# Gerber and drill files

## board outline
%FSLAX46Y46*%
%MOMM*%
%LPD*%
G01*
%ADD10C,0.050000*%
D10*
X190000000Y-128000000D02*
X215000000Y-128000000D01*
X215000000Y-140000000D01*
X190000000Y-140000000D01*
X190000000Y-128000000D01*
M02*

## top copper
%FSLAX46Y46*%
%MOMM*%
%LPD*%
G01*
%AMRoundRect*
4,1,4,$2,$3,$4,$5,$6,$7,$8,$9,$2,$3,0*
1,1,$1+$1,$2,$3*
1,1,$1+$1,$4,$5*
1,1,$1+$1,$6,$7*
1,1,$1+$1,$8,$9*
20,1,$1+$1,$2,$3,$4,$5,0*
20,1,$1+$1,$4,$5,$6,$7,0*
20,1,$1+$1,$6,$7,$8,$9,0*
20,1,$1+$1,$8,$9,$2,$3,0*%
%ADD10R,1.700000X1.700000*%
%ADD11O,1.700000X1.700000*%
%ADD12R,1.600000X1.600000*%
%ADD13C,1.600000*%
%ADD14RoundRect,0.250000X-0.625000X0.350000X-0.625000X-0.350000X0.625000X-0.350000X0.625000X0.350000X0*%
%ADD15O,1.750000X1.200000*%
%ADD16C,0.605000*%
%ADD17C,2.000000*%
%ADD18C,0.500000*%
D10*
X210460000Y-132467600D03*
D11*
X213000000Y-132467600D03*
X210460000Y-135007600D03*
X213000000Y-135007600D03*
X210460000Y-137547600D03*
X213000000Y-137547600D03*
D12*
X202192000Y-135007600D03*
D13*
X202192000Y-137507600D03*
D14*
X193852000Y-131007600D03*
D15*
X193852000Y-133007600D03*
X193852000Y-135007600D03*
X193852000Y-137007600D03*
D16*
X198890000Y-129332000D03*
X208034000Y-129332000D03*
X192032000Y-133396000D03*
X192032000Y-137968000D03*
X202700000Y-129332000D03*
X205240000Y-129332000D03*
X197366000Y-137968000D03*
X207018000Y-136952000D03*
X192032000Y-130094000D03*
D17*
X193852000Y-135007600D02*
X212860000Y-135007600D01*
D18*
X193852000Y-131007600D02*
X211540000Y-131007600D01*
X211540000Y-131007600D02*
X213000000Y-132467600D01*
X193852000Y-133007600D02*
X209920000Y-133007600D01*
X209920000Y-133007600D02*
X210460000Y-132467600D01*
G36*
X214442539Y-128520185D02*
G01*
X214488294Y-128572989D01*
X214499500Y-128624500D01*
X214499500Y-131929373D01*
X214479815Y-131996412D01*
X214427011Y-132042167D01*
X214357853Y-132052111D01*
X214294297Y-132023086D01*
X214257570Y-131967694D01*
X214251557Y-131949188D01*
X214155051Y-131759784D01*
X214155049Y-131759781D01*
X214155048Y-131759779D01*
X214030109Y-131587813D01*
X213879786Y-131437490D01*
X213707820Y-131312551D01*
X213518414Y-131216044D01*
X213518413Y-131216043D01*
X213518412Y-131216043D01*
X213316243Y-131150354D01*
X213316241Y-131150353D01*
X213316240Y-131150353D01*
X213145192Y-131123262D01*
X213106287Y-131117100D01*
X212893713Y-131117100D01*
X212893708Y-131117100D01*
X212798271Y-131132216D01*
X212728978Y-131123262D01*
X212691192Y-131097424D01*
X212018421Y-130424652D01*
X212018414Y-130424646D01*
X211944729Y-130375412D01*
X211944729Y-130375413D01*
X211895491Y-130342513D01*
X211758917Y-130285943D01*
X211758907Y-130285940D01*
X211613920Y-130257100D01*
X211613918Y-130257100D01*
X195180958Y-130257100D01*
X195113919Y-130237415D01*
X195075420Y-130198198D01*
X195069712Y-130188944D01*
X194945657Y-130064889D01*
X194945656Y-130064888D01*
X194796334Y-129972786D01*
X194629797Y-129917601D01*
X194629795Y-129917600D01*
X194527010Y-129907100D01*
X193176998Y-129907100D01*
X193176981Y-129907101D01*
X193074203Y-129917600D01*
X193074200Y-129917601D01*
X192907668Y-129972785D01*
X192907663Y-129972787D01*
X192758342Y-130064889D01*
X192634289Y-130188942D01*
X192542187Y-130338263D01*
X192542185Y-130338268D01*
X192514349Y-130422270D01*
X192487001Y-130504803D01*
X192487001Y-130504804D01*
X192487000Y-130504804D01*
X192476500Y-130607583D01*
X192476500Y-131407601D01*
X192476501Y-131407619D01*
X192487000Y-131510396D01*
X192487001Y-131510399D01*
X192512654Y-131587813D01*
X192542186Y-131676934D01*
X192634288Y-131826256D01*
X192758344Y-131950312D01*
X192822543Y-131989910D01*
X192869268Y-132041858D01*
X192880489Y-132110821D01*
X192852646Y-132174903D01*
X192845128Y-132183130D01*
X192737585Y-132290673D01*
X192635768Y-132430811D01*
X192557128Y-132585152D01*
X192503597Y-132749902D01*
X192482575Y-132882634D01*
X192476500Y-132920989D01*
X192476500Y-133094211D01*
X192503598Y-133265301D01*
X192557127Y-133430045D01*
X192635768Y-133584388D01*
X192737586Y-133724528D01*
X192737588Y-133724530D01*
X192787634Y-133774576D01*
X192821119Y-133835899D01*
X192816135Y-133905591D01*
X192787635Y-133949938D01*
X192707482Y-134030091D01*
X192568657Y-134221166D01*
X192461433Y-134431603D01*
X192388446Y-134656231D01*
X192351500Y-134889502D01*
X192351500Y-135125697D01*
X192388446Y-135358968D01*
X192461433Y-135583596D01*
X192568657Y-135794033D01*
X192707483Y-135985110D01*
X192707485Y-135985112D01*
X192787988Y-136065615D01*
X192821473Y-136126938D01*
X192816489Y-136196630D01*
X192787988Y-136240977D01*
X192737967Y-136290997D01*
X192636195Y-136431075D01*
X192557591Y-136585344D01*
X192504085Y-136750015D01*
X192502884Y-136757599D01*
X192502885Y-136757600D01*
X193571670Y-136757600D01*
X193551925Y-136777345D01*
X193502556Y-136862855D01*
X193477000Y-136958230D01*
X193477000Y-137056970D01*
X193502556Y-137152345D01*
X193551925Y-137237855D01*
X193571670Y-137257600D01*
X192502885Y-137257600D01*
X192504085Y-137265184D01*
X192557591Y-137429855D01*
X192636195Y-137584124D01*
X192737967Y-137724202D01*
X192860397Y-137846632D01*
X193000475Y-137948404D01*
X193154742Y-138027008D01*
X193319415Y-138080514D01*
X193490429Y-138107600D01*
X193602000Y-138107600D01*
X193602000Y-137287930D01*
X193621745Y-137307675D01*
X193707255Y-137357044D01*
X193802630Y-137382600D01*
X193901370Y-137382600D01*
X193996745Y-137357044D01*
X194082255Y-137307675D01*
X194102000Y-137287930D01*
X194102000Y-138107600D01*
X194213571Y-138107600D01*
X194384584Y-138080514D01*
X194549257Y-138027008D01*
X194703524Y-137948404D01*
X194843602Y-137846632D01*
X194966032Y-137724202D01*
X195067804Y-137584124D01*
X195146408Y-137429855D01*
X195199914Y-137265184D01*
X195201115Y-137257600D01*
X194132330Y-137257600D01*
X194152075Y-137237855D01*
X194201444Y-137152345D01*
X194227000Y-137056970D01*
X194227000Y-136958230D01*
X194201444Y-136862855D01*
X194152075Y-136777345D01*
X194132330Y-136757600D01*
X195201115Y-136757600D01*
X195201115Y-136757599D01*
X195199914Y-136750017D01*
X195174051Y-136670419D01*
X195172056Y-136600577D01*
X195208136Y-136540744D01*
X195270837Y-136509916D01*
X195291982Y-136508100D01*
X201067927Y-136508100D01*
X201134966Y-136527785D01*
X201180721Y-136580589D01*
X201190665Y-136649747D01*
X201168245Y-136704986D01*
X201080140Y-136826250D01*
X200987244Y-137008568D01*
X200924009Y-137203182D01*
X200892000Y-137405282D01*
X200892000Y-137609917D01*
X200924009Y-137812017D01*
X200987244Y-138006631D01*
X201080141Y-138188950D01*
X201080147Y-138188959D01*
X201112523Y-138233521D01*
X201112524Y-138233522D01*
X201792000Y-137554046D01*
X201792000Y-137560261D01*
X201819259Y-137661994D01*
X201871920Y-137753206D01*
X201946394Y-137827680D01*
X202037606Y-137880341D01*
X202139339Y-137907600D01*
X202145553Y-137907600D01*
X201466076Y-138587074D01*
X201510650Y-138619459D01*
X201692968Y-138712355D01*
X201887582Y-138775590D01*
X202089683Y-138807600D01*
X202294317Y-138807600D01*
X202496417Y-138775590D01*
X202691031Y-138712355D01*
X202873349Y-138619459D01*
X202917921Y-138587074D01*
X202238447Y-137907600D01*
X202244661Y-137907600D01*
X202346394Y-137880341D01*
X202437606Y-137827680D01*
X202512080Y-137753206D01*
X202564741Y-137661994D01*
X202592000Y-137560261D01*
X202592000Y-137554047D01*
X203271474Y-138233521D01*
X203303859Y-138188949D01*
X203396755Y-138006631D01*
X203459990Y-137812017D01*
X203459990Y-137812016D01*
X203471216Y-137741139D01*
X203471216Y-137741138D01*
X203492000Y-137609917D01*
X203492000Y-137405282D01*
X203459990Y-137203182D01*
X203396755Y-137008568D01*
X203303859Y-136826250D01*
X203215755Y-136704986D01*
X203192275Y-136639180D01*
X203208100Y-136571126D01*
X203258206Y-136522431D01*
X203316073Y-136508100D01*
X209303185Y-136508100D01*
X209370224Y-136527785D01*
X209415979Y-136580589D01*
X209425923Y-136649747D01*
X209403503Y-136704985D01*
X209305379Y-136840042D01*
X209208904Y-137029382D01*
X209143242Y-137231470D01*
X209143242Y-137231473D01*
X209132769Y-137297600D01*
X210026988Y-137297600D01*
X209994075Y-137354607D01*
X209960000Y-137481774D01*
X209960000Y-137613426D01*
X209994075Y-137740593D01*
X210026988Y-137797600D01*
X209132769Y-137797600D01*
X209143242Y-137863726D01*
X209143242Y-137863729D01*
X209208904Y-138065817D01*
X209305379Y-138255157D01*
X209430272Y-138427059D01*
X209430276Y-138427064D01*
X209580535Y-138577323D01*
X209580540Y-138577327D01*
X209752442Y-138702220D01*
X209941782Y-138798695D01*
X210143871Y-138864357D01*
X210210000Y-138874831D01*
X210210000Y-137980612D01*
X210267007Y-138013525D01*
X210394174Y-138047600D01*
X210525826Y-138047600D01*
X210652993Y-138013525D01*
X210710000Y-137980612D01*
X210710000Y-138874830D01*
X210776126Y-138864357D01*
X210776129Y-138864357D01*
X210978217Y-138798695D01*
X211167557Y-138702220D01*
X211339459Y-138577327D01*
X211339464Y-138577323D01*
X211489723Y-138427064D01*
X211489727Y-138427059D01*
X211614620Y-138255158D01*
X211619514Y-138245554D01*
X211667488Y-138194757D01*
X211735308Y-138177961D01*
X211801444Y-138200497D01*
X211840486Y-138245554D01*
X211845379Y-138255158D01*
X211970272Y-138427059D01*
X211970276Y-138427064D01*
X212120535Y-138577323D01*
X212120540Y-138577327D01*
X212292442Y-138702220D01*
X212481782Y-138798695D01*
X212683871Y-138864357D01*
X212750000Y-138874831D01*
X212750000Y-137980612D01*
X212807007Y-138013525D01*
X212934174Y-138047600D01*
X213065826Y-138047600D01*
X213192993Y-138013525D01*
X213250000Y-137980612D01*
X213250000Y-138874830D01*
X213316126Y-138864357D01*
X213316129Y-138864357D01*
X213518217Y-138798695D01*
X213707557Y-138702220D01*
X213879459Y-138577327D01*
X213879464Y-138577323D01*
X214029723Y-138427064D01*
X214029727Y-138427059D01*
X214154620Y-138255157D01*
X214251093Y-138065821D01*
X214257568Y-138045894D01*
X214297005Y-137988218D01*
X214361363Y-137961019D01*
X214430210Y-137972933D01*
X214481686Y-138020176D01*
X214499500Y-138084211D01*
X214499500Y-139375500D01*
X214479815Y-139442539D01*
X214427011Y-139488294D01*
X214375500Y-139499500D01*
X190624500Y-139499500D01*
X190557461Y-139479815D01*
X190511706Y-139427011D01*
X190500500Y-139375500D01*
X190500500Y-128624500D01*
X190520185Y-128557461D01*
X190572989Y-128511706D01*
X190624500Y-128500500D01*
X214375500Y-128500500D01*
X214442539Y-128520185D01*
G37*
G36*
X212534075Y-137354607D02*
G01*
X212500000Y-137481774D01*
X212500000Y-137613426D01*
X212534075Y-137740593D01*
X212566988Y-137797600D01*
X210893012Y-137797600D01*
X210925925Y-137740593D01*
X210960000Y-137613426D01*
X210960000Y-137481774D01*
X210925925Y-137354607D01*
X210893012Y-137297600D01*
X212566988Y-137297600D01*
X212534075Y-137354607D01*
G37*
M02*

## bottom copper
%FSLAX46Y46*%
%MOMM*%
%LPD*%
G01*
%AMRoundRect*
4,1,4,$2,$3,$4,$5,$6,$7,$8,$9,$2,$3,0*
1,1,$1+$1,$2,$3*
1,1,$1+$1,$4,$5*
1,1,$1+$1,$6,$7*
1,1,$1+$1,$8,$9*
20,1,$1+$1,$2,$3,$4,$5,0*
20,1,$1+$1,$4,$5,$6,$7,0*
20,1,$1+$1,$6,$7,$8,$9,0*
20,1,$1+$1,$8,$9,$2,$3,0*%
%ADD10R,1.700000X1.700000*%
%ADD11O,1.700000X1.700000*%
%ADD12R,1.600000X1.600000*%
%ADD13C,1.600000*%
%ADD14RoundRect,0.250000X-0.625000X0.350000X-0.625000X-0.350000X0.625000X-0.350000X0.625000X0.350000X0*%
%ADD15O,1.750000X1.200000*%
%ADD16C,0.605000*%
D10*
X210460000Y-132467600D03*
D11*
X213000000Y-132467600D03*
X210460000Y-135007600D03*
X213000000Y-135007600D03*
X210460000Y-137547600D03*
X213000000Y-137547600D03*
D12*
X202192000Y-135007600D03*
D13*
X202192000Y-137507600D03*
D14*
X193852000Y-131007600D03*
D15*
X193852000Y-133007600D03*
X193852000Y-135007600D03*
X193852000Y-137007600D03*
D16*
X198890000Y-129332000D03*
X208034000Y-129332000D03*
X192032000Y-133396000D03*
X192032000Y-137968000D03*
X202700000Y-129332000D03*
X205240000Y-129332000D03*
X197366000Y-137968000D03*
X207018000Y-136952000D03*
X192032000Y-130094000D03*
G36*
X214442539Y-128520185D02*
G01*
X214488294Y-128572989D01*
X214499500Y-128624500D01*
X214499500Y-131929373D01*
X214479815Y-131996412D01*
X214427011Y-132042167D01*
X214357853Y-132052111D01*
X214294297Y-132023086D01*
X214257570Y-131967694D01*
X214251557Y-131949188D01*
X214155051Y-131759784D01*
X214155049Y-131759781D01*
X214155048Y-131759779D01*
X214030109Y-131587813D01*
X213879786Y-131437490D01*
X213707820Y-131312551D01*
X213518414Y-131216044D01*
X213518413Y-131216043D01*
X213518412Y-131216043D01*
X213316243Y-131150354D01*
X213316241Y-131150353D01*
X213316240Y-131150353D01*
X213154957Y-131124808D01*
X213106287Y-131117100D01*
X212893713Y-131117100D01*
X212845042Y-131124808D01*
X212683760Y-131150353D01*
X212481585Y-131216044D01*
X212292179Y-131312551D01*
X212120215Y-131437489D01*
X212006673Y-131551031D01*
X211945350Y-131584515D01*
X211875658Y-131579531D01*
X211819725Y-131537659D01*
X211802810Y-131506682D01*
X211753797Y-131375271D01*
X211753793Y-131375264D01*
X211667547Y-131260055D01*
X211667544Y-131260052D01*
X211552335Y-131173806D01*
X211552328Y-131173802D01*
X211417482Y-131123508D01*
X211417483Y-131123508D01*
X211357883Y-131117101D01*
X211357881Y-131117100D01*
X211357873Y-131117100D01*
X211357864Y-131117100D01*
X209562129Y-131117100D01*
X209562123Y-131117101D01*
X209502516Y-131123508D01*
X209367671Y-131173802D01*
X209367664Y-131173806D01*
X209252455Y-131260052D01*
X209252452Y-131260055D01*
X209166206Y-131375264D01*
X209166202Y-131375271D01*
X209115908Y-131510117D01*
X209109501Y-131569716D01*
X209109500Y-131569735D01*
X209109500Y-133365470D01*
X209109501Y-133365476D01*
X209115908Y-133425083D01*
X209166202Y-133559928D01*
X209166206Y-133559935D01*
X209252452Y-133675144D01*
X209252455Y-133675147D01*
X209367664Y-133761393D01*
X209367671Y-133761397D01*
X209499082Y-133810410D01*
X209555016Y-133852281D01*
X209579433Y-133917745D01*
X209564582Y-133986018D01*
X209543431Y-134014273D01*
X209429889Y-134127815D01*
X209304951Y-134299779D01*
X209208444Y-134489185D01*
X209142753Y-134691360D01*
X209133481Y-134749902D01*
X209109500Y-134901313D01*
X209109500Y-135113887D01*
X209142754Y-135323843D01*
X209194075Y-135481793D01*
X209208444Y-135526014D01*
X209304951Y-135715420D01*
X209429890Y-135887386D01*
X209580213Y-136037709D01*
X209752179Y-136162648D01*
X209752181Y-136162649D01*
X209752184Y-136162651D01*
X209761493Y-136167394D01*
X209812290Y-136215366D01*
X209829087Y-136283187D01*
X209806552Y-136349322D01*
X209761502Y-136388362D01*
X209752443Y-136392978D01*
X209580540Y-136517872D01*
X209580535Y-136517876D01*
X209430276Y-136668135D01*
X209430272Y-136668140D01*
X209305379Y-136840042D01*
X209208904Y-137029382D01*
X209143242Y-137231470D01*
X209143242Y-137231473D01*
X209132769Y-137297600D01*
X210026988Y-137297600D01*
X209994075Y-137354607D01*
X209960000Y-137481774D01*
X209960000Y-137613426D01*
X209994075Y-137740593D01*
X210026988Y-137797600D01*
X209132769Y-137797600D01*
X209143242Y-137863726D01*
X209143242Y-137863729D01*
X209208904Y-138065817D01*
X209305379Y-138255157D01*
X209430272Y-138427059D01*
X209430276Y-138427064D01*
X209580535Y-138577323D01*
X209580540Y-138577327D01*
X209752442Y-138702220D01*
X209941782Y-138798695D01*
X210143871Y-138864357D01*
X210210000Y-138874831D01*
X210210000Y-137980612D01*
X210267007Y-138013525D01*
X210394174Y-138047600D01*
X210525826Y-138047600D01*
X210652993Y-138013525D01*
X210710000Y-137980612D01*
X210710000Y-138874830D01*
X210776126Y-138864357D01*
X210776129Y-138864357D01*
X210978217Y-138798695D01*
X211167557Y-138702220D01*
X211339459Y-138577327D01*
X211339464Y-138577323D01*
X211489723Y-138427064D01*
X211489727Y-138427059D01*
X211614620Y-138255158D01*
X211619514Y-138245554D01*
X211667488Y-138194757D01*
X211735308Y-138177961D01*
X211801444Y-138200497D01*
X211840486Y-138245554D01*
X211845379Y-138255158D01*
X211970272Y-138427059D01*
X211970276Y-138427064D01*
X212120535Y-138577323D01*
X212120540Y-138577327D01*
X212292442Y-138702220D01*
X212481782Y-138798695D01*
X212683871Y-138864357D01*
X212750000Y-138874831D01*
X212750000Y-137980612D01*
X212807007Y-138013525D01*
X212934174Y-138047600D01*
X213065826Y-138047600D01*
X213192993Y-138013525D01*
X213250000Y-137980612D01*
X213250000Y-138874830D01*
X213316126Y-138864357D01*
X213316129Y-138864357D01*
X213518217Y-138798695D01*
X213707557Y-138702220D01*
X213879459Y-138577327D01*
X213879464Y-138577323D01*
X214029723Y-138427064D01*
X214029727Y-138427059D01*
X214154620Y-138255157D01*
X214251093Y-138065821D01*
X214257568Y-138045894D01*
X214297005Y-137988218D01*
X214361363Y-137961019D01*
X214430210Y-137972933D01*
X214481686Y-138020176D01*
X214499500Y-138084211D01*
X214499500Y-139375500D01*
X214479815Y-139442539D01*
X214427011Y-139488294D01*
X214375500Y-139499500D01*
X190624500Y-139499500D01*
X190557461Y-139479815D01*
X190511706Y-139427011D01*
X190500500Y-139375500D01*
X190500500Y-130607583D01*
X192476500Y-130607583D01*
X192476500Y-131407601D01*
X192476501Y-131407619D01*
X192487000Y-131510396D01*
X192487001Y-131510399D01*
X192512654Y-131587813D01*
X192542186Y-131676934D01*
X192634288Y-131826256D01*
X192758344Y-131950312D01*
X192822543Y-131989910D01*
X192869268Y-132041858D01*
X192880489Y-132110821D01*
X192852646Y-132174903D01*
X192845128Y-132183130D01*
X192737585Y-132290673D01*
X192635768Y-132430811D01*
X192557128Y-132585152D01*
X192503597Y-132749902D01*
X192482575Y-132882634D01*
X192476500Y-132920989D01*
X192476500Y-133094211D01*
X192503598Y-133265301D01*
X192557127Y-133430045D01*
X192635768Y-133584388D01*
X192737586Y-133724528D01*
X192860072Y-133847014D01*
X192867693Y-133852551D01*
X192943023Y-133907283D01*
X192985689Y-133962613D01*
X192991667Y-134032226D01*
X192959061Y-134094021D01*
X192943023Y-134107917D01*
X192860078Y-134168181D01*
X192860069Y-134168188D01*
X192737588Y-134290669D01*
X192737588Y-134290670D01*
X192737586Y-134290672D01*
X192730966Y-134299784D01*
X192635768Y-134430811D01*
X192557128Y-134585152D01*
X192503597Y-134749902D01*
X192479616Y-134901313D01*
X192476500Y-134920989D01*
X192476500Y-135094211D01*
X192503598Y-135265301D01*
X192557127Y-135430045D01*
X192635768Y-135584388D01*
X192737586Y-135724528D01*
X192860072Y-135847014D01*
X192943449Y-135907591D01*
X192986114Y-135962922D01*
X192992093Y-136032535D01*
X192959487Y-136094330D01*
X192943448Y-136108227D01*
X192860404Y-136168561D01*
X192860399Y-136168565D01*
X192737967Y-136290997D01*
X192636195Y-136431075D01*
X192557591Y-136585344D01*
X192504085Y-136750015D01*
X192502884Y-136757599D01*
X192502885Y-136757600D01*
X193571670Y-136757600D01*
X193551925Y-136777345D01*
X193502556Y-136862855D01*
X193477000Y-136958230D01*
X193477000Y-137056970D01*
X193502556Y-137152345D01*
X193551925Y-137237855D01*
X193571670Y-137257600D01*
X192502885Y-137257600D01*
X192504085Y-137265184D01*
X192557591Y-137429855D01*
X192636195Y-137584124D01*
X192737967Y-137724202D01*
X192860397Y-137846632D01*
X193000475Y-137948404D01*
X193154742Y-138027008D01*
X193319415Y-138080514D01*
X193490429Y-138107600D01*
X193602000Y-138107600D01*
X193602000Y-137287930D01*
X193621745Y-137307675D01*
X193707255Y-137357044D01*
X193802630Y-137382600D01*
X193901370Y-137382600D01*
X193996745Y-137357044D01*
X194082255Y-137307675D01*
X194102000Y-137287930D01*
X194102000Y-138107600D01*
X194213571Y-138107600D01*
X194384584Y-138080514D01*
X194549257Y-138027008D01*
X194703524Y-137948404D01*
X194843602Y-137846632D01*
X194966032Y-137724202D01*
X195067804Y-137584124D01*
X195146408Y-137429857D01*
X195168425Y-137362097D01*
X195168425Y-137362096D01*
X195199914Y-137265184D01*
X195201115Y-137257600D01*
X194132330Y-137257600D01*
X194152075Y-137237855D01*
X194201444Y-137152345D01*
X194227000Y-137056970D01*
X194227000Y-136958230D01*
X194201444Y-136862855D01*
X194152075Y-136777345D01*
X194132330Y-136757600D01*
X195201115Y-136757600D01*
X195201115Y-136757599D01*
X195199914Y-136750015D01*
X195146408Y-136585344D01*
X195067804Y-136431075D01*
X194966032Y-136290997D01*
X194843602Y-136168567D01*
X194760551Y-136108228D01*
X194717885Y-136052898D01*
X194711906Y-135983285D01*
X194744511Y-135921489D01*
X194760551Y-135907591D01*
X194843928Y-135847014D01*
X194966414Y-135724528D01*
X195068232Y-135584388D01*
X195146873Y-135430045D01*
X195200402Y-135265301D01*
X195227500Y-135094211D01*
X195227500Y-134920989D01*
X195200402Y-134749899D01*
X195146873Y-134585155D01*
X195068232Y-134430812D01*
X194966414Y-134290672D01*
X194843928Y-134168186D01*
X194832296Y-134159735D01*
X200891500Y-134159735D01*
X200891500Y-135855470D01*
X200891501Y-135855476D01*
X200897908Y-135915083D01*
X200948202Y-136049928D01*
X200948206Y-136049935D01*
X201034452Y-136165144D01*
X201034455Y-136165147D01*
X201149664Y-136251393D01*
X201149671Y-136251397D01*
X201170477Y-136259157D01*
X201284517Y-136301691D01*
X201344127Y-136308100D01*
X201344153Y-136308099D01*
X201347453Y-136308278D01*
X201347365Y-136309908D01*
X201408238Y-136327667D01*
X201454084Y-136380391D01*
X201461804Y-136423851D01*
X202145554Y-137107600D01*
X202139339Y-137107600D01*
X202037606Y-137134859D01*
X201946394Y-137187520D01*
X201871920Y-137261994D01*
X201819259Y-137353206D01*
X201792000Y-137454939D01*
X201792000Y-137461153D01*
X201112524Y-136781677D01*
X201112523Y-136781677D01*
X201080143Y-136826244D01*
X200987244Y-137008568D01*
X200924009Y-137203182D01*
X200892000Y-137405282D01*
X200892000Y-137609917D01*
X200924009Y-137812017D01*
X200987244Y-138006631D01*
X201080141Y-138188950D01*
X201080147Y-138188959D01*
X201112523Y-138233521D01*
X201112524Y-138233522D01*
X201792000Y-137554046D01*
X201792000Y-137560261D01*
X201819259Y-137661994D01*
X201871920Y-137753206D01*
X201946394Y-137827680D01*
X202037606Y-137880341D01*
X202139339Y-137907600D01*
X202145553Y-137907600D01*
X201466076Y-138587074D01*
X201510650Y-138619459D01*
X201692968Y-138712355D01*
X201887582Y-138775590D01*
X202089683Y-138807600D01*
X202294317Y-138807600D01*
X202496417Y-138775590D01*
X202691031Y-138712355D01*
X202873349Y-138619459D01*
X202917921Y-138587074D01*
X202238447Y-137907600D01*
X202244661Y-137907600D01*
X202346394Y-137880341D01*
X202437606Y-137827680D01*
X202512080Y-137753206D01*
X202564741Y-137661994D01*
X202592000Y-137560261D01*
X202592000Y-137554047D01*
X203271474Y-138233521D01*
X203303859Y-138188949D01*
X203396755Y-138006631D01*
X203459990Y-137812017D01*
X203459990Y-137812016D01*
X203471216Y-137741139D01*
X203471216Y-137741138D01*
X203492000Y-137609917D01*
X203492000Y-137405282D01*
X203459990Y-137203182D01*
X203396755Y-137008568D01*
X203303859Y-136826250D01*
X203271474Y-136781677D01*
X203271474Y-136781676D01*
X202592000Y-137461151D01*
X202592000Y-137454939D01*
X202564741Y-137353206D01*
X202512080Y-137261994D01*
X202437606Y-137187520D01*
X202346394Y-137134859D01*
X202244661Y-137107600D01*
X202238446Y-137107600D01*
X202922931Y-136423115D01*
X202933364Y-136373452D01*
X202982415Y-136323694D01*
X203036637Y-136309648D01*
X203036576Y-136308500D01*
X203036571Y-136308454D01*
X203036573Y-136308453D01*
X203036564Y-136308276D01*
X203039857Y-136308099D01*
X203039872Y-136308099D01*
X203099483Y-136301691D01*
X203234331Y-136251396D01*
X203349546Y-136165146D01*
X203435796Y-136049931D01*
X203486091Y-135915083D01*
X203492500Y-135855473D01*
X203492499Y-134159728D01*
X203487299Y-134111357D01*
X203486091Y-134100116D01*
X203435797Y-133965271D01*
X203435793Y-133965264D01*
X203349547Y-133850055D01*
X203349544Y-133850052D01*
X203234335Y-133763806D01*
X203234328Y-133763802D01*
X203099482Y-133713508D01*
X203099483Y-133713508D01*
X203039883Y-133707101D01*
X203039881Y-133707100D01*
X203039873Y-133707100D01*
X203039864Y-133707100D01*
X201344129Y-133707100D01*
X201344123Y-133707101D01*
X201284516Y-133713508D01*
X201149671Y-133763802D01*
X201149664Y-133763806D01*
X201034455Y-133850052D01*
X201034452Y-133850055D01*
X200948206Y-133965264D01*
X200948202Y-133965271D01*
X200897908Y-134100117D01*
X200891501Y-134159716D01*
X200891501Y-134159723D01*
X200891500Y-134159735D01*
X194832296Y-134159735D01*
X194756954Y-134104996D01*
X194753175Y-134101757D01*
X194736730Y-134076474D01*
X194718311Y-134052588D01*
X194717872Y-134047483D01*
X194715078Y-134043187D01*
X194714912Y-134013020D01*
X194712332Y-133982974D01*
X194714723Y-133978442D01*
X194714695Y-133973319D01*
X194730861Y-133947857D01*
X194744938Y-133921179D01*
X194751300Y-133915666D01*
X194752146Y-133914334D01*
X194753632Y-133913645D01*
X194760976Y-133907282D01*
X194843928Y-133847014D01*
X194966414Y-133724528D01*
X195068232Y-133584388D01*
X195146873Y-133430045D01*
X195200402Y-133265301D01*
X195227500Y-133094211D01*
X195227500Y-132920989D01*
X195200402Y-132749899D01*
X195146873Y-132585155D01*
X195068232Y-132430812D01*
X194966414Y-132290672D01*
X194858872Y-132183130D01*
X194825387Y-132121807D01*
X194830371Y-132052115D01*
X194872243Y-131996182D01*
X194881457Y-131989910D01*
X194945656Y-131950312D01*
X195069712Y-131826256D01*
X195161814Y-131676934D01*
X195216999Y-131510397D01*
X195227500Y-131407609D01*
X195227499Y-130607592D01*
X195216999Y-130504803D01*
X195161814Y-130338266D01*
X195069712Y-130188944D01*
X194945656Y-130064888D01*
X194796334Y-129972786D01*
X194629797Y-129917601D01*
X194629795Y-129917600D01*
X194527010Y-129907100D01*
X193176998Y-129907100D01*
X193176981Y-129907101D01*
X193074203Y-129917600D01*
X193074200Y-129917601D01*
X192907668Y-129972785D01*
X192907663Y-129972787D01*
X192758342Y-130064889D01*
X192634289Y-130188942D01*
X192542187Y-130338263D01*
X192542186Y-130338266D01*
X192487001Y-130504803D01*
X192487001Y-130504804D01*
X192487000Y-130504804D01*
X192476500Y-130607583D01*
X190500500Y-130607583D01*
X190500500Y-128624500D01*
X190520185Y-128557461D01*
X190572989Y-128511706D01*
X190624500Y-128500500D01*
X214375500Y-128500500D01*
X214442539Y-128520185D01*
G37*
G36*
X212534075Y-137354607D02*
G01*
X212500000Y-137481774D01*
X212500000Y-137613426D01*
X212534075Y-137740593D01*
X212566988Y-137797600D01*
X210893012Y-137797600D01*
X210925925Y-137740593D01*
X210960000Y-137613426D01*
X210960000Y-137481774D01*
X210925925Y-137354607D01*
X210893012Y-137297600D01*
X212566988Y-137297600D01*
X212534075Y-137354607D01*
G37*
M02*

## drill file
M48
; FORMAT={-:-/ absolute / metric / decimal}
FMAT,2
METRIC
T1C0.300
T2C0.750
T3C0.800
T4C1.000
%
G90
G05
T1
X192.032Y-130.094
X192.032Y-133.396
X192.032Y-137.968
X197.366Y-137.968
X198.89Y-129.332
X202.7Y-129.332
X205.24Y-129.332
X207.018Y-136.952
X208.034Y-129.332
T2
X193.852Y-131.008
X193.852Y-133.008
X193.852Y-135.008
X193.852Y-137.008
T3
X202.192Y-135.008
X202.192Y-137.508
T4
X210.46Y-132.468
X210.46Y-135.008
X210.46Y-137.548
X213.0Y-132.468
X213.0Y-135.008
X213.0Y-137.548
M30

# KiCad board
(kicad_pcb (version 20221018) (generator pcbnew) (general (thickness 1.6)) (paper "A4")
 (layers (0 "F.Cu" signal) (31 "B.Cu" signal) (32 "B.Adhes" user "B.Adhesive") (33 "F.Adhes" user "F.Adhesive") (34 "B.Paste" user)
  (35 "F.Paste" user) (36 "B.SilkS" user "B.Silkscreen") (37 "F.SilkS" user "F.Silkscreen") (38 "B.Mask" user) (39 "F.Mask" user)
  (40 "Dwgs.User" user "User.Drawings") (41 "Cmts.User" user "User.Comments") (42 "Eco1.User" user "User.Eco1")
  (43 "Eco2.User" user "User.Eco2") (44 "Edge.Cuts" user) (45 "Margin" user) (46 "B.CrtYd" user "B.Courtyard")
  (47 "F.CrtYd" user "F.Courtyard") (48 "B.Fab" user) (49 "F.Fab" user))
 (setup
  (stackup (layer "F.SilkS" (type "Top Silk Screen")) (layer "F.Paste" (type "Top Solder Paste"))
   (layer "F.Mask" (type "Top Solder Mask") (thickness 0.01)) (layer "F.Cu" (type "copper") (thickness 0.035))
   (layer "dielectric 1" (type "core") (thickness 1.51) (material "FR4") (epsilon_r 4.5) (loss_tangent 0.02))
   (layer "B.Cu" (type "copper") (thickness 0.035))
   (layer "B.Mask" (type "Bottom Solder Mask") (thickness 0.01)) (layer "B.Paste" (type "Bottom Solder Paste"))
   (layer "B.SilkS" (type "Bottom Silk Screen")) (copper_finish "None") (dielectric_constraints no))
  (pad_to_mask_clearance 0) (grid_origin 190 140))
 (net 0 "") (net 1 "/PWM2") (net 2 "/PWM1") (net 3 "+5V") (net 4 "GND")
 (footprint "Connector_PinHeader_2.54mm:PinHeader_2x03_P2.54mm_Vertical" (layer "F.Cu") (at 210.46 132.4676)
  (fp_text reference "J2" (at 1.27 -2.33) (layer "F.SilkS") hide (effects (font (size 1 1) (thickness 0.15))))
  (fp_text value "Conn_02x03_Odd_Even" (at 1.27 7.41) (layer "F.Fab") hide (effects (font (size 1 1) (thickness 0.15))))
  (pad "1" thru_hole rect (at 0 0) (size 1.7 1.7) (drill 1) (layers "*.Cu" "*.Mask") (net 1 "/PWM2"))
  (pad "2" thru_hole oval (at 2.54 0) (size 1.7 1.7) (drill 1) (layers "*.Cu" "*.Mask") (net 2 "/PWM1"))
  (pad "3" thru_hole oval (at 0 2.54) (size 1.7 1.7) (drill 1) (layers "*.Cu" "*.Mask") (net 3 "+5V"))
  (pad "4" thru_hole oval (at 2.54 2.54) (size 1.7 1.7) (drill 1) (layers "*.Cu" "*.Mask") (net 3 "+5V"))
  (pad "5" thru_hole oval (at 0 5.08) (size 1.7 1.7) (drill 1) (layers "*.Cu" "*.Mask") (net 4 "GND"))
  (pad "6" thru_hole oval (at 2.54 5.08) (size 1.7 1.7) (drill 1) (layers "*.Cu" "*.Mask") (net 4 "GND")))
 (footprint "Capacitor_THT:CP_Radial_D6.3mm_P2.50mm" (layer "F.Cu") (at 202.192 135.0076 -90)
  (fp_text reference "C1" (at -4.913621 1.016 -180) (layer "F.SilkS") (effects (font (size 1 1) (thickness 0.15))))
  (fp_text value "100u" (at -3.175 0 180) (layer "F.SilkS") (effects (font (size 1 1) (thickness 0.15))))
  (pad "1" thru_hole rect (at 0 0 270) (size 1.6 1.6) (drill 0.8) (layers "*.Cu" "*.Mask") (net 3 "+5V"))
  (pad "2" thru_hole circle (at 2.5 0 270) (size 1.6 1.6) (drill 0.8) (layers "*.Cu" "*.Mask") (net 4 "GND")))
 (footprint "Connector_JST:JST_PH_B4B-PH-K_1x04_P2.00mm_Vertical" (layer "F.Cu") (at 193.852 131.0076 -90)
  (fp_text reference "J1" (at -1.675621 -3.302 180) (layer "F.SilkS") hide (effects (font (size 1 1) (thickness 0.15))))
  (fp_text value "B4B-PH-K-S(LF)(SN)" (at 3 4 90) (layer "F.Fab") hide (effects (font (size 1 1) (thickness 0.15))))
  (pad "1" thru_hole roundrect (at 0 0 270) (size 1.2 1.75) (drill 0.75) (layers "*.Cu" "*.Mask") (roundrect_rratio 0.2083333333)
   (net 2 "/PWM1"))
  (pad "2" thru_hole oval (at 2 0 270) (size 1.2 1.75) (drill 0.75) (layers "*.Cu" "*.Mask") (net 1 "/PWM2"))
  (pad "3" thru_hole oval (at 4 0 270) (size 1.2 1.75) (drill 0.75) (layers "*.Cu" "*.Mask") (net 3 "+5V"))
  (pad "4" thru_hole oval (at 6 0 270) (size 1.2 1.75) (drill 0.75) (layers "*.Cu" "*.Mask") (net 4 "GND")))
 (gr_rect (start 190 128) (end 215 140) (stroke (width 0.05) (type default)) (fill none) (layer "Edge.Cuts"))
 (segment (start 193.852 135.0076) (end 212.86 135.0076) (width 2) (layer "F.Cu") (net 3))
 (via (at 198.89 129.332) (size 0.605) (drill 0.3) (layers "F.Cu" "B.Cu") (free) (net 4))
 (via (at 208.034 129.332) (size 0.605) (drill 0.3) (layers "F.Cu" "B.Cu") (free) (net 4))
 (via (at 192.032 133.396) (size 0.605) (drill 0.3) (layers "F.Cu" "B.Cu") (free) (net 4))
 (via (at 192.032 137.968) (size 0.605) (drill 0.3) (layers "F.Cu" "B.Cu") (free) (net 4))
 (via (at 202.7 129.332) (size 0.605) (drill 0.3) (layers "F.Cu" "B.Cu") (free) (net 4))
 (via (at 205.24 129.332) (size 0.605) (drill 0.3) (layers "F.Cu" "B.Cu") (free) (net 4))
 (via (at 197.366 137.968) (size 0.605) (drill 0.3) (layers "F.Cu" "B.Cu") (free) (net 4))
 (via (at 207.018 136.952) (size 0.605) (drill 0.3) (layers "F.Cu" "B.Cu") (free) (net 4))
 (via (at 192.032 130.094) (size 0.605) (drill 0.3) (layers "F.Cu" "B.Cu") (free) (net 4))
 (segment (start 193.852 131.0076) (end 211.54 131.0076) (width 0.5) (layer "F.Cu") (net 2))
 (segment (start 211.54 131.0076) (end 213 132.4676) (width 0.5) (layer "F.Cu") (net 2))
 (segment (start 193.852 133.0076) (end 209.92 133.0076) (width 0.5) (layer "F.Cu") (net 1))
 (segment (start 209.92 133.0076) (end 210.46 132.4676) (width 0.5) (layer "F.Cu") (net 1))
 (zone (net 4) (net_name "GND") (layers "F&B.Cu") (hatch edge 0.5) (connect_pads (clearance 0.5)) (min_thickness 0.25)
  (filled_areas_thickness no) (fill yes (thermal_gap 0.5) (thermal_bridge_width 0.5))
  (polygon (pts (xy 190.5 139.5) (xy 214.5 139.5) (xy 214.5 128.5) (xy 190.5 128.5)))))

